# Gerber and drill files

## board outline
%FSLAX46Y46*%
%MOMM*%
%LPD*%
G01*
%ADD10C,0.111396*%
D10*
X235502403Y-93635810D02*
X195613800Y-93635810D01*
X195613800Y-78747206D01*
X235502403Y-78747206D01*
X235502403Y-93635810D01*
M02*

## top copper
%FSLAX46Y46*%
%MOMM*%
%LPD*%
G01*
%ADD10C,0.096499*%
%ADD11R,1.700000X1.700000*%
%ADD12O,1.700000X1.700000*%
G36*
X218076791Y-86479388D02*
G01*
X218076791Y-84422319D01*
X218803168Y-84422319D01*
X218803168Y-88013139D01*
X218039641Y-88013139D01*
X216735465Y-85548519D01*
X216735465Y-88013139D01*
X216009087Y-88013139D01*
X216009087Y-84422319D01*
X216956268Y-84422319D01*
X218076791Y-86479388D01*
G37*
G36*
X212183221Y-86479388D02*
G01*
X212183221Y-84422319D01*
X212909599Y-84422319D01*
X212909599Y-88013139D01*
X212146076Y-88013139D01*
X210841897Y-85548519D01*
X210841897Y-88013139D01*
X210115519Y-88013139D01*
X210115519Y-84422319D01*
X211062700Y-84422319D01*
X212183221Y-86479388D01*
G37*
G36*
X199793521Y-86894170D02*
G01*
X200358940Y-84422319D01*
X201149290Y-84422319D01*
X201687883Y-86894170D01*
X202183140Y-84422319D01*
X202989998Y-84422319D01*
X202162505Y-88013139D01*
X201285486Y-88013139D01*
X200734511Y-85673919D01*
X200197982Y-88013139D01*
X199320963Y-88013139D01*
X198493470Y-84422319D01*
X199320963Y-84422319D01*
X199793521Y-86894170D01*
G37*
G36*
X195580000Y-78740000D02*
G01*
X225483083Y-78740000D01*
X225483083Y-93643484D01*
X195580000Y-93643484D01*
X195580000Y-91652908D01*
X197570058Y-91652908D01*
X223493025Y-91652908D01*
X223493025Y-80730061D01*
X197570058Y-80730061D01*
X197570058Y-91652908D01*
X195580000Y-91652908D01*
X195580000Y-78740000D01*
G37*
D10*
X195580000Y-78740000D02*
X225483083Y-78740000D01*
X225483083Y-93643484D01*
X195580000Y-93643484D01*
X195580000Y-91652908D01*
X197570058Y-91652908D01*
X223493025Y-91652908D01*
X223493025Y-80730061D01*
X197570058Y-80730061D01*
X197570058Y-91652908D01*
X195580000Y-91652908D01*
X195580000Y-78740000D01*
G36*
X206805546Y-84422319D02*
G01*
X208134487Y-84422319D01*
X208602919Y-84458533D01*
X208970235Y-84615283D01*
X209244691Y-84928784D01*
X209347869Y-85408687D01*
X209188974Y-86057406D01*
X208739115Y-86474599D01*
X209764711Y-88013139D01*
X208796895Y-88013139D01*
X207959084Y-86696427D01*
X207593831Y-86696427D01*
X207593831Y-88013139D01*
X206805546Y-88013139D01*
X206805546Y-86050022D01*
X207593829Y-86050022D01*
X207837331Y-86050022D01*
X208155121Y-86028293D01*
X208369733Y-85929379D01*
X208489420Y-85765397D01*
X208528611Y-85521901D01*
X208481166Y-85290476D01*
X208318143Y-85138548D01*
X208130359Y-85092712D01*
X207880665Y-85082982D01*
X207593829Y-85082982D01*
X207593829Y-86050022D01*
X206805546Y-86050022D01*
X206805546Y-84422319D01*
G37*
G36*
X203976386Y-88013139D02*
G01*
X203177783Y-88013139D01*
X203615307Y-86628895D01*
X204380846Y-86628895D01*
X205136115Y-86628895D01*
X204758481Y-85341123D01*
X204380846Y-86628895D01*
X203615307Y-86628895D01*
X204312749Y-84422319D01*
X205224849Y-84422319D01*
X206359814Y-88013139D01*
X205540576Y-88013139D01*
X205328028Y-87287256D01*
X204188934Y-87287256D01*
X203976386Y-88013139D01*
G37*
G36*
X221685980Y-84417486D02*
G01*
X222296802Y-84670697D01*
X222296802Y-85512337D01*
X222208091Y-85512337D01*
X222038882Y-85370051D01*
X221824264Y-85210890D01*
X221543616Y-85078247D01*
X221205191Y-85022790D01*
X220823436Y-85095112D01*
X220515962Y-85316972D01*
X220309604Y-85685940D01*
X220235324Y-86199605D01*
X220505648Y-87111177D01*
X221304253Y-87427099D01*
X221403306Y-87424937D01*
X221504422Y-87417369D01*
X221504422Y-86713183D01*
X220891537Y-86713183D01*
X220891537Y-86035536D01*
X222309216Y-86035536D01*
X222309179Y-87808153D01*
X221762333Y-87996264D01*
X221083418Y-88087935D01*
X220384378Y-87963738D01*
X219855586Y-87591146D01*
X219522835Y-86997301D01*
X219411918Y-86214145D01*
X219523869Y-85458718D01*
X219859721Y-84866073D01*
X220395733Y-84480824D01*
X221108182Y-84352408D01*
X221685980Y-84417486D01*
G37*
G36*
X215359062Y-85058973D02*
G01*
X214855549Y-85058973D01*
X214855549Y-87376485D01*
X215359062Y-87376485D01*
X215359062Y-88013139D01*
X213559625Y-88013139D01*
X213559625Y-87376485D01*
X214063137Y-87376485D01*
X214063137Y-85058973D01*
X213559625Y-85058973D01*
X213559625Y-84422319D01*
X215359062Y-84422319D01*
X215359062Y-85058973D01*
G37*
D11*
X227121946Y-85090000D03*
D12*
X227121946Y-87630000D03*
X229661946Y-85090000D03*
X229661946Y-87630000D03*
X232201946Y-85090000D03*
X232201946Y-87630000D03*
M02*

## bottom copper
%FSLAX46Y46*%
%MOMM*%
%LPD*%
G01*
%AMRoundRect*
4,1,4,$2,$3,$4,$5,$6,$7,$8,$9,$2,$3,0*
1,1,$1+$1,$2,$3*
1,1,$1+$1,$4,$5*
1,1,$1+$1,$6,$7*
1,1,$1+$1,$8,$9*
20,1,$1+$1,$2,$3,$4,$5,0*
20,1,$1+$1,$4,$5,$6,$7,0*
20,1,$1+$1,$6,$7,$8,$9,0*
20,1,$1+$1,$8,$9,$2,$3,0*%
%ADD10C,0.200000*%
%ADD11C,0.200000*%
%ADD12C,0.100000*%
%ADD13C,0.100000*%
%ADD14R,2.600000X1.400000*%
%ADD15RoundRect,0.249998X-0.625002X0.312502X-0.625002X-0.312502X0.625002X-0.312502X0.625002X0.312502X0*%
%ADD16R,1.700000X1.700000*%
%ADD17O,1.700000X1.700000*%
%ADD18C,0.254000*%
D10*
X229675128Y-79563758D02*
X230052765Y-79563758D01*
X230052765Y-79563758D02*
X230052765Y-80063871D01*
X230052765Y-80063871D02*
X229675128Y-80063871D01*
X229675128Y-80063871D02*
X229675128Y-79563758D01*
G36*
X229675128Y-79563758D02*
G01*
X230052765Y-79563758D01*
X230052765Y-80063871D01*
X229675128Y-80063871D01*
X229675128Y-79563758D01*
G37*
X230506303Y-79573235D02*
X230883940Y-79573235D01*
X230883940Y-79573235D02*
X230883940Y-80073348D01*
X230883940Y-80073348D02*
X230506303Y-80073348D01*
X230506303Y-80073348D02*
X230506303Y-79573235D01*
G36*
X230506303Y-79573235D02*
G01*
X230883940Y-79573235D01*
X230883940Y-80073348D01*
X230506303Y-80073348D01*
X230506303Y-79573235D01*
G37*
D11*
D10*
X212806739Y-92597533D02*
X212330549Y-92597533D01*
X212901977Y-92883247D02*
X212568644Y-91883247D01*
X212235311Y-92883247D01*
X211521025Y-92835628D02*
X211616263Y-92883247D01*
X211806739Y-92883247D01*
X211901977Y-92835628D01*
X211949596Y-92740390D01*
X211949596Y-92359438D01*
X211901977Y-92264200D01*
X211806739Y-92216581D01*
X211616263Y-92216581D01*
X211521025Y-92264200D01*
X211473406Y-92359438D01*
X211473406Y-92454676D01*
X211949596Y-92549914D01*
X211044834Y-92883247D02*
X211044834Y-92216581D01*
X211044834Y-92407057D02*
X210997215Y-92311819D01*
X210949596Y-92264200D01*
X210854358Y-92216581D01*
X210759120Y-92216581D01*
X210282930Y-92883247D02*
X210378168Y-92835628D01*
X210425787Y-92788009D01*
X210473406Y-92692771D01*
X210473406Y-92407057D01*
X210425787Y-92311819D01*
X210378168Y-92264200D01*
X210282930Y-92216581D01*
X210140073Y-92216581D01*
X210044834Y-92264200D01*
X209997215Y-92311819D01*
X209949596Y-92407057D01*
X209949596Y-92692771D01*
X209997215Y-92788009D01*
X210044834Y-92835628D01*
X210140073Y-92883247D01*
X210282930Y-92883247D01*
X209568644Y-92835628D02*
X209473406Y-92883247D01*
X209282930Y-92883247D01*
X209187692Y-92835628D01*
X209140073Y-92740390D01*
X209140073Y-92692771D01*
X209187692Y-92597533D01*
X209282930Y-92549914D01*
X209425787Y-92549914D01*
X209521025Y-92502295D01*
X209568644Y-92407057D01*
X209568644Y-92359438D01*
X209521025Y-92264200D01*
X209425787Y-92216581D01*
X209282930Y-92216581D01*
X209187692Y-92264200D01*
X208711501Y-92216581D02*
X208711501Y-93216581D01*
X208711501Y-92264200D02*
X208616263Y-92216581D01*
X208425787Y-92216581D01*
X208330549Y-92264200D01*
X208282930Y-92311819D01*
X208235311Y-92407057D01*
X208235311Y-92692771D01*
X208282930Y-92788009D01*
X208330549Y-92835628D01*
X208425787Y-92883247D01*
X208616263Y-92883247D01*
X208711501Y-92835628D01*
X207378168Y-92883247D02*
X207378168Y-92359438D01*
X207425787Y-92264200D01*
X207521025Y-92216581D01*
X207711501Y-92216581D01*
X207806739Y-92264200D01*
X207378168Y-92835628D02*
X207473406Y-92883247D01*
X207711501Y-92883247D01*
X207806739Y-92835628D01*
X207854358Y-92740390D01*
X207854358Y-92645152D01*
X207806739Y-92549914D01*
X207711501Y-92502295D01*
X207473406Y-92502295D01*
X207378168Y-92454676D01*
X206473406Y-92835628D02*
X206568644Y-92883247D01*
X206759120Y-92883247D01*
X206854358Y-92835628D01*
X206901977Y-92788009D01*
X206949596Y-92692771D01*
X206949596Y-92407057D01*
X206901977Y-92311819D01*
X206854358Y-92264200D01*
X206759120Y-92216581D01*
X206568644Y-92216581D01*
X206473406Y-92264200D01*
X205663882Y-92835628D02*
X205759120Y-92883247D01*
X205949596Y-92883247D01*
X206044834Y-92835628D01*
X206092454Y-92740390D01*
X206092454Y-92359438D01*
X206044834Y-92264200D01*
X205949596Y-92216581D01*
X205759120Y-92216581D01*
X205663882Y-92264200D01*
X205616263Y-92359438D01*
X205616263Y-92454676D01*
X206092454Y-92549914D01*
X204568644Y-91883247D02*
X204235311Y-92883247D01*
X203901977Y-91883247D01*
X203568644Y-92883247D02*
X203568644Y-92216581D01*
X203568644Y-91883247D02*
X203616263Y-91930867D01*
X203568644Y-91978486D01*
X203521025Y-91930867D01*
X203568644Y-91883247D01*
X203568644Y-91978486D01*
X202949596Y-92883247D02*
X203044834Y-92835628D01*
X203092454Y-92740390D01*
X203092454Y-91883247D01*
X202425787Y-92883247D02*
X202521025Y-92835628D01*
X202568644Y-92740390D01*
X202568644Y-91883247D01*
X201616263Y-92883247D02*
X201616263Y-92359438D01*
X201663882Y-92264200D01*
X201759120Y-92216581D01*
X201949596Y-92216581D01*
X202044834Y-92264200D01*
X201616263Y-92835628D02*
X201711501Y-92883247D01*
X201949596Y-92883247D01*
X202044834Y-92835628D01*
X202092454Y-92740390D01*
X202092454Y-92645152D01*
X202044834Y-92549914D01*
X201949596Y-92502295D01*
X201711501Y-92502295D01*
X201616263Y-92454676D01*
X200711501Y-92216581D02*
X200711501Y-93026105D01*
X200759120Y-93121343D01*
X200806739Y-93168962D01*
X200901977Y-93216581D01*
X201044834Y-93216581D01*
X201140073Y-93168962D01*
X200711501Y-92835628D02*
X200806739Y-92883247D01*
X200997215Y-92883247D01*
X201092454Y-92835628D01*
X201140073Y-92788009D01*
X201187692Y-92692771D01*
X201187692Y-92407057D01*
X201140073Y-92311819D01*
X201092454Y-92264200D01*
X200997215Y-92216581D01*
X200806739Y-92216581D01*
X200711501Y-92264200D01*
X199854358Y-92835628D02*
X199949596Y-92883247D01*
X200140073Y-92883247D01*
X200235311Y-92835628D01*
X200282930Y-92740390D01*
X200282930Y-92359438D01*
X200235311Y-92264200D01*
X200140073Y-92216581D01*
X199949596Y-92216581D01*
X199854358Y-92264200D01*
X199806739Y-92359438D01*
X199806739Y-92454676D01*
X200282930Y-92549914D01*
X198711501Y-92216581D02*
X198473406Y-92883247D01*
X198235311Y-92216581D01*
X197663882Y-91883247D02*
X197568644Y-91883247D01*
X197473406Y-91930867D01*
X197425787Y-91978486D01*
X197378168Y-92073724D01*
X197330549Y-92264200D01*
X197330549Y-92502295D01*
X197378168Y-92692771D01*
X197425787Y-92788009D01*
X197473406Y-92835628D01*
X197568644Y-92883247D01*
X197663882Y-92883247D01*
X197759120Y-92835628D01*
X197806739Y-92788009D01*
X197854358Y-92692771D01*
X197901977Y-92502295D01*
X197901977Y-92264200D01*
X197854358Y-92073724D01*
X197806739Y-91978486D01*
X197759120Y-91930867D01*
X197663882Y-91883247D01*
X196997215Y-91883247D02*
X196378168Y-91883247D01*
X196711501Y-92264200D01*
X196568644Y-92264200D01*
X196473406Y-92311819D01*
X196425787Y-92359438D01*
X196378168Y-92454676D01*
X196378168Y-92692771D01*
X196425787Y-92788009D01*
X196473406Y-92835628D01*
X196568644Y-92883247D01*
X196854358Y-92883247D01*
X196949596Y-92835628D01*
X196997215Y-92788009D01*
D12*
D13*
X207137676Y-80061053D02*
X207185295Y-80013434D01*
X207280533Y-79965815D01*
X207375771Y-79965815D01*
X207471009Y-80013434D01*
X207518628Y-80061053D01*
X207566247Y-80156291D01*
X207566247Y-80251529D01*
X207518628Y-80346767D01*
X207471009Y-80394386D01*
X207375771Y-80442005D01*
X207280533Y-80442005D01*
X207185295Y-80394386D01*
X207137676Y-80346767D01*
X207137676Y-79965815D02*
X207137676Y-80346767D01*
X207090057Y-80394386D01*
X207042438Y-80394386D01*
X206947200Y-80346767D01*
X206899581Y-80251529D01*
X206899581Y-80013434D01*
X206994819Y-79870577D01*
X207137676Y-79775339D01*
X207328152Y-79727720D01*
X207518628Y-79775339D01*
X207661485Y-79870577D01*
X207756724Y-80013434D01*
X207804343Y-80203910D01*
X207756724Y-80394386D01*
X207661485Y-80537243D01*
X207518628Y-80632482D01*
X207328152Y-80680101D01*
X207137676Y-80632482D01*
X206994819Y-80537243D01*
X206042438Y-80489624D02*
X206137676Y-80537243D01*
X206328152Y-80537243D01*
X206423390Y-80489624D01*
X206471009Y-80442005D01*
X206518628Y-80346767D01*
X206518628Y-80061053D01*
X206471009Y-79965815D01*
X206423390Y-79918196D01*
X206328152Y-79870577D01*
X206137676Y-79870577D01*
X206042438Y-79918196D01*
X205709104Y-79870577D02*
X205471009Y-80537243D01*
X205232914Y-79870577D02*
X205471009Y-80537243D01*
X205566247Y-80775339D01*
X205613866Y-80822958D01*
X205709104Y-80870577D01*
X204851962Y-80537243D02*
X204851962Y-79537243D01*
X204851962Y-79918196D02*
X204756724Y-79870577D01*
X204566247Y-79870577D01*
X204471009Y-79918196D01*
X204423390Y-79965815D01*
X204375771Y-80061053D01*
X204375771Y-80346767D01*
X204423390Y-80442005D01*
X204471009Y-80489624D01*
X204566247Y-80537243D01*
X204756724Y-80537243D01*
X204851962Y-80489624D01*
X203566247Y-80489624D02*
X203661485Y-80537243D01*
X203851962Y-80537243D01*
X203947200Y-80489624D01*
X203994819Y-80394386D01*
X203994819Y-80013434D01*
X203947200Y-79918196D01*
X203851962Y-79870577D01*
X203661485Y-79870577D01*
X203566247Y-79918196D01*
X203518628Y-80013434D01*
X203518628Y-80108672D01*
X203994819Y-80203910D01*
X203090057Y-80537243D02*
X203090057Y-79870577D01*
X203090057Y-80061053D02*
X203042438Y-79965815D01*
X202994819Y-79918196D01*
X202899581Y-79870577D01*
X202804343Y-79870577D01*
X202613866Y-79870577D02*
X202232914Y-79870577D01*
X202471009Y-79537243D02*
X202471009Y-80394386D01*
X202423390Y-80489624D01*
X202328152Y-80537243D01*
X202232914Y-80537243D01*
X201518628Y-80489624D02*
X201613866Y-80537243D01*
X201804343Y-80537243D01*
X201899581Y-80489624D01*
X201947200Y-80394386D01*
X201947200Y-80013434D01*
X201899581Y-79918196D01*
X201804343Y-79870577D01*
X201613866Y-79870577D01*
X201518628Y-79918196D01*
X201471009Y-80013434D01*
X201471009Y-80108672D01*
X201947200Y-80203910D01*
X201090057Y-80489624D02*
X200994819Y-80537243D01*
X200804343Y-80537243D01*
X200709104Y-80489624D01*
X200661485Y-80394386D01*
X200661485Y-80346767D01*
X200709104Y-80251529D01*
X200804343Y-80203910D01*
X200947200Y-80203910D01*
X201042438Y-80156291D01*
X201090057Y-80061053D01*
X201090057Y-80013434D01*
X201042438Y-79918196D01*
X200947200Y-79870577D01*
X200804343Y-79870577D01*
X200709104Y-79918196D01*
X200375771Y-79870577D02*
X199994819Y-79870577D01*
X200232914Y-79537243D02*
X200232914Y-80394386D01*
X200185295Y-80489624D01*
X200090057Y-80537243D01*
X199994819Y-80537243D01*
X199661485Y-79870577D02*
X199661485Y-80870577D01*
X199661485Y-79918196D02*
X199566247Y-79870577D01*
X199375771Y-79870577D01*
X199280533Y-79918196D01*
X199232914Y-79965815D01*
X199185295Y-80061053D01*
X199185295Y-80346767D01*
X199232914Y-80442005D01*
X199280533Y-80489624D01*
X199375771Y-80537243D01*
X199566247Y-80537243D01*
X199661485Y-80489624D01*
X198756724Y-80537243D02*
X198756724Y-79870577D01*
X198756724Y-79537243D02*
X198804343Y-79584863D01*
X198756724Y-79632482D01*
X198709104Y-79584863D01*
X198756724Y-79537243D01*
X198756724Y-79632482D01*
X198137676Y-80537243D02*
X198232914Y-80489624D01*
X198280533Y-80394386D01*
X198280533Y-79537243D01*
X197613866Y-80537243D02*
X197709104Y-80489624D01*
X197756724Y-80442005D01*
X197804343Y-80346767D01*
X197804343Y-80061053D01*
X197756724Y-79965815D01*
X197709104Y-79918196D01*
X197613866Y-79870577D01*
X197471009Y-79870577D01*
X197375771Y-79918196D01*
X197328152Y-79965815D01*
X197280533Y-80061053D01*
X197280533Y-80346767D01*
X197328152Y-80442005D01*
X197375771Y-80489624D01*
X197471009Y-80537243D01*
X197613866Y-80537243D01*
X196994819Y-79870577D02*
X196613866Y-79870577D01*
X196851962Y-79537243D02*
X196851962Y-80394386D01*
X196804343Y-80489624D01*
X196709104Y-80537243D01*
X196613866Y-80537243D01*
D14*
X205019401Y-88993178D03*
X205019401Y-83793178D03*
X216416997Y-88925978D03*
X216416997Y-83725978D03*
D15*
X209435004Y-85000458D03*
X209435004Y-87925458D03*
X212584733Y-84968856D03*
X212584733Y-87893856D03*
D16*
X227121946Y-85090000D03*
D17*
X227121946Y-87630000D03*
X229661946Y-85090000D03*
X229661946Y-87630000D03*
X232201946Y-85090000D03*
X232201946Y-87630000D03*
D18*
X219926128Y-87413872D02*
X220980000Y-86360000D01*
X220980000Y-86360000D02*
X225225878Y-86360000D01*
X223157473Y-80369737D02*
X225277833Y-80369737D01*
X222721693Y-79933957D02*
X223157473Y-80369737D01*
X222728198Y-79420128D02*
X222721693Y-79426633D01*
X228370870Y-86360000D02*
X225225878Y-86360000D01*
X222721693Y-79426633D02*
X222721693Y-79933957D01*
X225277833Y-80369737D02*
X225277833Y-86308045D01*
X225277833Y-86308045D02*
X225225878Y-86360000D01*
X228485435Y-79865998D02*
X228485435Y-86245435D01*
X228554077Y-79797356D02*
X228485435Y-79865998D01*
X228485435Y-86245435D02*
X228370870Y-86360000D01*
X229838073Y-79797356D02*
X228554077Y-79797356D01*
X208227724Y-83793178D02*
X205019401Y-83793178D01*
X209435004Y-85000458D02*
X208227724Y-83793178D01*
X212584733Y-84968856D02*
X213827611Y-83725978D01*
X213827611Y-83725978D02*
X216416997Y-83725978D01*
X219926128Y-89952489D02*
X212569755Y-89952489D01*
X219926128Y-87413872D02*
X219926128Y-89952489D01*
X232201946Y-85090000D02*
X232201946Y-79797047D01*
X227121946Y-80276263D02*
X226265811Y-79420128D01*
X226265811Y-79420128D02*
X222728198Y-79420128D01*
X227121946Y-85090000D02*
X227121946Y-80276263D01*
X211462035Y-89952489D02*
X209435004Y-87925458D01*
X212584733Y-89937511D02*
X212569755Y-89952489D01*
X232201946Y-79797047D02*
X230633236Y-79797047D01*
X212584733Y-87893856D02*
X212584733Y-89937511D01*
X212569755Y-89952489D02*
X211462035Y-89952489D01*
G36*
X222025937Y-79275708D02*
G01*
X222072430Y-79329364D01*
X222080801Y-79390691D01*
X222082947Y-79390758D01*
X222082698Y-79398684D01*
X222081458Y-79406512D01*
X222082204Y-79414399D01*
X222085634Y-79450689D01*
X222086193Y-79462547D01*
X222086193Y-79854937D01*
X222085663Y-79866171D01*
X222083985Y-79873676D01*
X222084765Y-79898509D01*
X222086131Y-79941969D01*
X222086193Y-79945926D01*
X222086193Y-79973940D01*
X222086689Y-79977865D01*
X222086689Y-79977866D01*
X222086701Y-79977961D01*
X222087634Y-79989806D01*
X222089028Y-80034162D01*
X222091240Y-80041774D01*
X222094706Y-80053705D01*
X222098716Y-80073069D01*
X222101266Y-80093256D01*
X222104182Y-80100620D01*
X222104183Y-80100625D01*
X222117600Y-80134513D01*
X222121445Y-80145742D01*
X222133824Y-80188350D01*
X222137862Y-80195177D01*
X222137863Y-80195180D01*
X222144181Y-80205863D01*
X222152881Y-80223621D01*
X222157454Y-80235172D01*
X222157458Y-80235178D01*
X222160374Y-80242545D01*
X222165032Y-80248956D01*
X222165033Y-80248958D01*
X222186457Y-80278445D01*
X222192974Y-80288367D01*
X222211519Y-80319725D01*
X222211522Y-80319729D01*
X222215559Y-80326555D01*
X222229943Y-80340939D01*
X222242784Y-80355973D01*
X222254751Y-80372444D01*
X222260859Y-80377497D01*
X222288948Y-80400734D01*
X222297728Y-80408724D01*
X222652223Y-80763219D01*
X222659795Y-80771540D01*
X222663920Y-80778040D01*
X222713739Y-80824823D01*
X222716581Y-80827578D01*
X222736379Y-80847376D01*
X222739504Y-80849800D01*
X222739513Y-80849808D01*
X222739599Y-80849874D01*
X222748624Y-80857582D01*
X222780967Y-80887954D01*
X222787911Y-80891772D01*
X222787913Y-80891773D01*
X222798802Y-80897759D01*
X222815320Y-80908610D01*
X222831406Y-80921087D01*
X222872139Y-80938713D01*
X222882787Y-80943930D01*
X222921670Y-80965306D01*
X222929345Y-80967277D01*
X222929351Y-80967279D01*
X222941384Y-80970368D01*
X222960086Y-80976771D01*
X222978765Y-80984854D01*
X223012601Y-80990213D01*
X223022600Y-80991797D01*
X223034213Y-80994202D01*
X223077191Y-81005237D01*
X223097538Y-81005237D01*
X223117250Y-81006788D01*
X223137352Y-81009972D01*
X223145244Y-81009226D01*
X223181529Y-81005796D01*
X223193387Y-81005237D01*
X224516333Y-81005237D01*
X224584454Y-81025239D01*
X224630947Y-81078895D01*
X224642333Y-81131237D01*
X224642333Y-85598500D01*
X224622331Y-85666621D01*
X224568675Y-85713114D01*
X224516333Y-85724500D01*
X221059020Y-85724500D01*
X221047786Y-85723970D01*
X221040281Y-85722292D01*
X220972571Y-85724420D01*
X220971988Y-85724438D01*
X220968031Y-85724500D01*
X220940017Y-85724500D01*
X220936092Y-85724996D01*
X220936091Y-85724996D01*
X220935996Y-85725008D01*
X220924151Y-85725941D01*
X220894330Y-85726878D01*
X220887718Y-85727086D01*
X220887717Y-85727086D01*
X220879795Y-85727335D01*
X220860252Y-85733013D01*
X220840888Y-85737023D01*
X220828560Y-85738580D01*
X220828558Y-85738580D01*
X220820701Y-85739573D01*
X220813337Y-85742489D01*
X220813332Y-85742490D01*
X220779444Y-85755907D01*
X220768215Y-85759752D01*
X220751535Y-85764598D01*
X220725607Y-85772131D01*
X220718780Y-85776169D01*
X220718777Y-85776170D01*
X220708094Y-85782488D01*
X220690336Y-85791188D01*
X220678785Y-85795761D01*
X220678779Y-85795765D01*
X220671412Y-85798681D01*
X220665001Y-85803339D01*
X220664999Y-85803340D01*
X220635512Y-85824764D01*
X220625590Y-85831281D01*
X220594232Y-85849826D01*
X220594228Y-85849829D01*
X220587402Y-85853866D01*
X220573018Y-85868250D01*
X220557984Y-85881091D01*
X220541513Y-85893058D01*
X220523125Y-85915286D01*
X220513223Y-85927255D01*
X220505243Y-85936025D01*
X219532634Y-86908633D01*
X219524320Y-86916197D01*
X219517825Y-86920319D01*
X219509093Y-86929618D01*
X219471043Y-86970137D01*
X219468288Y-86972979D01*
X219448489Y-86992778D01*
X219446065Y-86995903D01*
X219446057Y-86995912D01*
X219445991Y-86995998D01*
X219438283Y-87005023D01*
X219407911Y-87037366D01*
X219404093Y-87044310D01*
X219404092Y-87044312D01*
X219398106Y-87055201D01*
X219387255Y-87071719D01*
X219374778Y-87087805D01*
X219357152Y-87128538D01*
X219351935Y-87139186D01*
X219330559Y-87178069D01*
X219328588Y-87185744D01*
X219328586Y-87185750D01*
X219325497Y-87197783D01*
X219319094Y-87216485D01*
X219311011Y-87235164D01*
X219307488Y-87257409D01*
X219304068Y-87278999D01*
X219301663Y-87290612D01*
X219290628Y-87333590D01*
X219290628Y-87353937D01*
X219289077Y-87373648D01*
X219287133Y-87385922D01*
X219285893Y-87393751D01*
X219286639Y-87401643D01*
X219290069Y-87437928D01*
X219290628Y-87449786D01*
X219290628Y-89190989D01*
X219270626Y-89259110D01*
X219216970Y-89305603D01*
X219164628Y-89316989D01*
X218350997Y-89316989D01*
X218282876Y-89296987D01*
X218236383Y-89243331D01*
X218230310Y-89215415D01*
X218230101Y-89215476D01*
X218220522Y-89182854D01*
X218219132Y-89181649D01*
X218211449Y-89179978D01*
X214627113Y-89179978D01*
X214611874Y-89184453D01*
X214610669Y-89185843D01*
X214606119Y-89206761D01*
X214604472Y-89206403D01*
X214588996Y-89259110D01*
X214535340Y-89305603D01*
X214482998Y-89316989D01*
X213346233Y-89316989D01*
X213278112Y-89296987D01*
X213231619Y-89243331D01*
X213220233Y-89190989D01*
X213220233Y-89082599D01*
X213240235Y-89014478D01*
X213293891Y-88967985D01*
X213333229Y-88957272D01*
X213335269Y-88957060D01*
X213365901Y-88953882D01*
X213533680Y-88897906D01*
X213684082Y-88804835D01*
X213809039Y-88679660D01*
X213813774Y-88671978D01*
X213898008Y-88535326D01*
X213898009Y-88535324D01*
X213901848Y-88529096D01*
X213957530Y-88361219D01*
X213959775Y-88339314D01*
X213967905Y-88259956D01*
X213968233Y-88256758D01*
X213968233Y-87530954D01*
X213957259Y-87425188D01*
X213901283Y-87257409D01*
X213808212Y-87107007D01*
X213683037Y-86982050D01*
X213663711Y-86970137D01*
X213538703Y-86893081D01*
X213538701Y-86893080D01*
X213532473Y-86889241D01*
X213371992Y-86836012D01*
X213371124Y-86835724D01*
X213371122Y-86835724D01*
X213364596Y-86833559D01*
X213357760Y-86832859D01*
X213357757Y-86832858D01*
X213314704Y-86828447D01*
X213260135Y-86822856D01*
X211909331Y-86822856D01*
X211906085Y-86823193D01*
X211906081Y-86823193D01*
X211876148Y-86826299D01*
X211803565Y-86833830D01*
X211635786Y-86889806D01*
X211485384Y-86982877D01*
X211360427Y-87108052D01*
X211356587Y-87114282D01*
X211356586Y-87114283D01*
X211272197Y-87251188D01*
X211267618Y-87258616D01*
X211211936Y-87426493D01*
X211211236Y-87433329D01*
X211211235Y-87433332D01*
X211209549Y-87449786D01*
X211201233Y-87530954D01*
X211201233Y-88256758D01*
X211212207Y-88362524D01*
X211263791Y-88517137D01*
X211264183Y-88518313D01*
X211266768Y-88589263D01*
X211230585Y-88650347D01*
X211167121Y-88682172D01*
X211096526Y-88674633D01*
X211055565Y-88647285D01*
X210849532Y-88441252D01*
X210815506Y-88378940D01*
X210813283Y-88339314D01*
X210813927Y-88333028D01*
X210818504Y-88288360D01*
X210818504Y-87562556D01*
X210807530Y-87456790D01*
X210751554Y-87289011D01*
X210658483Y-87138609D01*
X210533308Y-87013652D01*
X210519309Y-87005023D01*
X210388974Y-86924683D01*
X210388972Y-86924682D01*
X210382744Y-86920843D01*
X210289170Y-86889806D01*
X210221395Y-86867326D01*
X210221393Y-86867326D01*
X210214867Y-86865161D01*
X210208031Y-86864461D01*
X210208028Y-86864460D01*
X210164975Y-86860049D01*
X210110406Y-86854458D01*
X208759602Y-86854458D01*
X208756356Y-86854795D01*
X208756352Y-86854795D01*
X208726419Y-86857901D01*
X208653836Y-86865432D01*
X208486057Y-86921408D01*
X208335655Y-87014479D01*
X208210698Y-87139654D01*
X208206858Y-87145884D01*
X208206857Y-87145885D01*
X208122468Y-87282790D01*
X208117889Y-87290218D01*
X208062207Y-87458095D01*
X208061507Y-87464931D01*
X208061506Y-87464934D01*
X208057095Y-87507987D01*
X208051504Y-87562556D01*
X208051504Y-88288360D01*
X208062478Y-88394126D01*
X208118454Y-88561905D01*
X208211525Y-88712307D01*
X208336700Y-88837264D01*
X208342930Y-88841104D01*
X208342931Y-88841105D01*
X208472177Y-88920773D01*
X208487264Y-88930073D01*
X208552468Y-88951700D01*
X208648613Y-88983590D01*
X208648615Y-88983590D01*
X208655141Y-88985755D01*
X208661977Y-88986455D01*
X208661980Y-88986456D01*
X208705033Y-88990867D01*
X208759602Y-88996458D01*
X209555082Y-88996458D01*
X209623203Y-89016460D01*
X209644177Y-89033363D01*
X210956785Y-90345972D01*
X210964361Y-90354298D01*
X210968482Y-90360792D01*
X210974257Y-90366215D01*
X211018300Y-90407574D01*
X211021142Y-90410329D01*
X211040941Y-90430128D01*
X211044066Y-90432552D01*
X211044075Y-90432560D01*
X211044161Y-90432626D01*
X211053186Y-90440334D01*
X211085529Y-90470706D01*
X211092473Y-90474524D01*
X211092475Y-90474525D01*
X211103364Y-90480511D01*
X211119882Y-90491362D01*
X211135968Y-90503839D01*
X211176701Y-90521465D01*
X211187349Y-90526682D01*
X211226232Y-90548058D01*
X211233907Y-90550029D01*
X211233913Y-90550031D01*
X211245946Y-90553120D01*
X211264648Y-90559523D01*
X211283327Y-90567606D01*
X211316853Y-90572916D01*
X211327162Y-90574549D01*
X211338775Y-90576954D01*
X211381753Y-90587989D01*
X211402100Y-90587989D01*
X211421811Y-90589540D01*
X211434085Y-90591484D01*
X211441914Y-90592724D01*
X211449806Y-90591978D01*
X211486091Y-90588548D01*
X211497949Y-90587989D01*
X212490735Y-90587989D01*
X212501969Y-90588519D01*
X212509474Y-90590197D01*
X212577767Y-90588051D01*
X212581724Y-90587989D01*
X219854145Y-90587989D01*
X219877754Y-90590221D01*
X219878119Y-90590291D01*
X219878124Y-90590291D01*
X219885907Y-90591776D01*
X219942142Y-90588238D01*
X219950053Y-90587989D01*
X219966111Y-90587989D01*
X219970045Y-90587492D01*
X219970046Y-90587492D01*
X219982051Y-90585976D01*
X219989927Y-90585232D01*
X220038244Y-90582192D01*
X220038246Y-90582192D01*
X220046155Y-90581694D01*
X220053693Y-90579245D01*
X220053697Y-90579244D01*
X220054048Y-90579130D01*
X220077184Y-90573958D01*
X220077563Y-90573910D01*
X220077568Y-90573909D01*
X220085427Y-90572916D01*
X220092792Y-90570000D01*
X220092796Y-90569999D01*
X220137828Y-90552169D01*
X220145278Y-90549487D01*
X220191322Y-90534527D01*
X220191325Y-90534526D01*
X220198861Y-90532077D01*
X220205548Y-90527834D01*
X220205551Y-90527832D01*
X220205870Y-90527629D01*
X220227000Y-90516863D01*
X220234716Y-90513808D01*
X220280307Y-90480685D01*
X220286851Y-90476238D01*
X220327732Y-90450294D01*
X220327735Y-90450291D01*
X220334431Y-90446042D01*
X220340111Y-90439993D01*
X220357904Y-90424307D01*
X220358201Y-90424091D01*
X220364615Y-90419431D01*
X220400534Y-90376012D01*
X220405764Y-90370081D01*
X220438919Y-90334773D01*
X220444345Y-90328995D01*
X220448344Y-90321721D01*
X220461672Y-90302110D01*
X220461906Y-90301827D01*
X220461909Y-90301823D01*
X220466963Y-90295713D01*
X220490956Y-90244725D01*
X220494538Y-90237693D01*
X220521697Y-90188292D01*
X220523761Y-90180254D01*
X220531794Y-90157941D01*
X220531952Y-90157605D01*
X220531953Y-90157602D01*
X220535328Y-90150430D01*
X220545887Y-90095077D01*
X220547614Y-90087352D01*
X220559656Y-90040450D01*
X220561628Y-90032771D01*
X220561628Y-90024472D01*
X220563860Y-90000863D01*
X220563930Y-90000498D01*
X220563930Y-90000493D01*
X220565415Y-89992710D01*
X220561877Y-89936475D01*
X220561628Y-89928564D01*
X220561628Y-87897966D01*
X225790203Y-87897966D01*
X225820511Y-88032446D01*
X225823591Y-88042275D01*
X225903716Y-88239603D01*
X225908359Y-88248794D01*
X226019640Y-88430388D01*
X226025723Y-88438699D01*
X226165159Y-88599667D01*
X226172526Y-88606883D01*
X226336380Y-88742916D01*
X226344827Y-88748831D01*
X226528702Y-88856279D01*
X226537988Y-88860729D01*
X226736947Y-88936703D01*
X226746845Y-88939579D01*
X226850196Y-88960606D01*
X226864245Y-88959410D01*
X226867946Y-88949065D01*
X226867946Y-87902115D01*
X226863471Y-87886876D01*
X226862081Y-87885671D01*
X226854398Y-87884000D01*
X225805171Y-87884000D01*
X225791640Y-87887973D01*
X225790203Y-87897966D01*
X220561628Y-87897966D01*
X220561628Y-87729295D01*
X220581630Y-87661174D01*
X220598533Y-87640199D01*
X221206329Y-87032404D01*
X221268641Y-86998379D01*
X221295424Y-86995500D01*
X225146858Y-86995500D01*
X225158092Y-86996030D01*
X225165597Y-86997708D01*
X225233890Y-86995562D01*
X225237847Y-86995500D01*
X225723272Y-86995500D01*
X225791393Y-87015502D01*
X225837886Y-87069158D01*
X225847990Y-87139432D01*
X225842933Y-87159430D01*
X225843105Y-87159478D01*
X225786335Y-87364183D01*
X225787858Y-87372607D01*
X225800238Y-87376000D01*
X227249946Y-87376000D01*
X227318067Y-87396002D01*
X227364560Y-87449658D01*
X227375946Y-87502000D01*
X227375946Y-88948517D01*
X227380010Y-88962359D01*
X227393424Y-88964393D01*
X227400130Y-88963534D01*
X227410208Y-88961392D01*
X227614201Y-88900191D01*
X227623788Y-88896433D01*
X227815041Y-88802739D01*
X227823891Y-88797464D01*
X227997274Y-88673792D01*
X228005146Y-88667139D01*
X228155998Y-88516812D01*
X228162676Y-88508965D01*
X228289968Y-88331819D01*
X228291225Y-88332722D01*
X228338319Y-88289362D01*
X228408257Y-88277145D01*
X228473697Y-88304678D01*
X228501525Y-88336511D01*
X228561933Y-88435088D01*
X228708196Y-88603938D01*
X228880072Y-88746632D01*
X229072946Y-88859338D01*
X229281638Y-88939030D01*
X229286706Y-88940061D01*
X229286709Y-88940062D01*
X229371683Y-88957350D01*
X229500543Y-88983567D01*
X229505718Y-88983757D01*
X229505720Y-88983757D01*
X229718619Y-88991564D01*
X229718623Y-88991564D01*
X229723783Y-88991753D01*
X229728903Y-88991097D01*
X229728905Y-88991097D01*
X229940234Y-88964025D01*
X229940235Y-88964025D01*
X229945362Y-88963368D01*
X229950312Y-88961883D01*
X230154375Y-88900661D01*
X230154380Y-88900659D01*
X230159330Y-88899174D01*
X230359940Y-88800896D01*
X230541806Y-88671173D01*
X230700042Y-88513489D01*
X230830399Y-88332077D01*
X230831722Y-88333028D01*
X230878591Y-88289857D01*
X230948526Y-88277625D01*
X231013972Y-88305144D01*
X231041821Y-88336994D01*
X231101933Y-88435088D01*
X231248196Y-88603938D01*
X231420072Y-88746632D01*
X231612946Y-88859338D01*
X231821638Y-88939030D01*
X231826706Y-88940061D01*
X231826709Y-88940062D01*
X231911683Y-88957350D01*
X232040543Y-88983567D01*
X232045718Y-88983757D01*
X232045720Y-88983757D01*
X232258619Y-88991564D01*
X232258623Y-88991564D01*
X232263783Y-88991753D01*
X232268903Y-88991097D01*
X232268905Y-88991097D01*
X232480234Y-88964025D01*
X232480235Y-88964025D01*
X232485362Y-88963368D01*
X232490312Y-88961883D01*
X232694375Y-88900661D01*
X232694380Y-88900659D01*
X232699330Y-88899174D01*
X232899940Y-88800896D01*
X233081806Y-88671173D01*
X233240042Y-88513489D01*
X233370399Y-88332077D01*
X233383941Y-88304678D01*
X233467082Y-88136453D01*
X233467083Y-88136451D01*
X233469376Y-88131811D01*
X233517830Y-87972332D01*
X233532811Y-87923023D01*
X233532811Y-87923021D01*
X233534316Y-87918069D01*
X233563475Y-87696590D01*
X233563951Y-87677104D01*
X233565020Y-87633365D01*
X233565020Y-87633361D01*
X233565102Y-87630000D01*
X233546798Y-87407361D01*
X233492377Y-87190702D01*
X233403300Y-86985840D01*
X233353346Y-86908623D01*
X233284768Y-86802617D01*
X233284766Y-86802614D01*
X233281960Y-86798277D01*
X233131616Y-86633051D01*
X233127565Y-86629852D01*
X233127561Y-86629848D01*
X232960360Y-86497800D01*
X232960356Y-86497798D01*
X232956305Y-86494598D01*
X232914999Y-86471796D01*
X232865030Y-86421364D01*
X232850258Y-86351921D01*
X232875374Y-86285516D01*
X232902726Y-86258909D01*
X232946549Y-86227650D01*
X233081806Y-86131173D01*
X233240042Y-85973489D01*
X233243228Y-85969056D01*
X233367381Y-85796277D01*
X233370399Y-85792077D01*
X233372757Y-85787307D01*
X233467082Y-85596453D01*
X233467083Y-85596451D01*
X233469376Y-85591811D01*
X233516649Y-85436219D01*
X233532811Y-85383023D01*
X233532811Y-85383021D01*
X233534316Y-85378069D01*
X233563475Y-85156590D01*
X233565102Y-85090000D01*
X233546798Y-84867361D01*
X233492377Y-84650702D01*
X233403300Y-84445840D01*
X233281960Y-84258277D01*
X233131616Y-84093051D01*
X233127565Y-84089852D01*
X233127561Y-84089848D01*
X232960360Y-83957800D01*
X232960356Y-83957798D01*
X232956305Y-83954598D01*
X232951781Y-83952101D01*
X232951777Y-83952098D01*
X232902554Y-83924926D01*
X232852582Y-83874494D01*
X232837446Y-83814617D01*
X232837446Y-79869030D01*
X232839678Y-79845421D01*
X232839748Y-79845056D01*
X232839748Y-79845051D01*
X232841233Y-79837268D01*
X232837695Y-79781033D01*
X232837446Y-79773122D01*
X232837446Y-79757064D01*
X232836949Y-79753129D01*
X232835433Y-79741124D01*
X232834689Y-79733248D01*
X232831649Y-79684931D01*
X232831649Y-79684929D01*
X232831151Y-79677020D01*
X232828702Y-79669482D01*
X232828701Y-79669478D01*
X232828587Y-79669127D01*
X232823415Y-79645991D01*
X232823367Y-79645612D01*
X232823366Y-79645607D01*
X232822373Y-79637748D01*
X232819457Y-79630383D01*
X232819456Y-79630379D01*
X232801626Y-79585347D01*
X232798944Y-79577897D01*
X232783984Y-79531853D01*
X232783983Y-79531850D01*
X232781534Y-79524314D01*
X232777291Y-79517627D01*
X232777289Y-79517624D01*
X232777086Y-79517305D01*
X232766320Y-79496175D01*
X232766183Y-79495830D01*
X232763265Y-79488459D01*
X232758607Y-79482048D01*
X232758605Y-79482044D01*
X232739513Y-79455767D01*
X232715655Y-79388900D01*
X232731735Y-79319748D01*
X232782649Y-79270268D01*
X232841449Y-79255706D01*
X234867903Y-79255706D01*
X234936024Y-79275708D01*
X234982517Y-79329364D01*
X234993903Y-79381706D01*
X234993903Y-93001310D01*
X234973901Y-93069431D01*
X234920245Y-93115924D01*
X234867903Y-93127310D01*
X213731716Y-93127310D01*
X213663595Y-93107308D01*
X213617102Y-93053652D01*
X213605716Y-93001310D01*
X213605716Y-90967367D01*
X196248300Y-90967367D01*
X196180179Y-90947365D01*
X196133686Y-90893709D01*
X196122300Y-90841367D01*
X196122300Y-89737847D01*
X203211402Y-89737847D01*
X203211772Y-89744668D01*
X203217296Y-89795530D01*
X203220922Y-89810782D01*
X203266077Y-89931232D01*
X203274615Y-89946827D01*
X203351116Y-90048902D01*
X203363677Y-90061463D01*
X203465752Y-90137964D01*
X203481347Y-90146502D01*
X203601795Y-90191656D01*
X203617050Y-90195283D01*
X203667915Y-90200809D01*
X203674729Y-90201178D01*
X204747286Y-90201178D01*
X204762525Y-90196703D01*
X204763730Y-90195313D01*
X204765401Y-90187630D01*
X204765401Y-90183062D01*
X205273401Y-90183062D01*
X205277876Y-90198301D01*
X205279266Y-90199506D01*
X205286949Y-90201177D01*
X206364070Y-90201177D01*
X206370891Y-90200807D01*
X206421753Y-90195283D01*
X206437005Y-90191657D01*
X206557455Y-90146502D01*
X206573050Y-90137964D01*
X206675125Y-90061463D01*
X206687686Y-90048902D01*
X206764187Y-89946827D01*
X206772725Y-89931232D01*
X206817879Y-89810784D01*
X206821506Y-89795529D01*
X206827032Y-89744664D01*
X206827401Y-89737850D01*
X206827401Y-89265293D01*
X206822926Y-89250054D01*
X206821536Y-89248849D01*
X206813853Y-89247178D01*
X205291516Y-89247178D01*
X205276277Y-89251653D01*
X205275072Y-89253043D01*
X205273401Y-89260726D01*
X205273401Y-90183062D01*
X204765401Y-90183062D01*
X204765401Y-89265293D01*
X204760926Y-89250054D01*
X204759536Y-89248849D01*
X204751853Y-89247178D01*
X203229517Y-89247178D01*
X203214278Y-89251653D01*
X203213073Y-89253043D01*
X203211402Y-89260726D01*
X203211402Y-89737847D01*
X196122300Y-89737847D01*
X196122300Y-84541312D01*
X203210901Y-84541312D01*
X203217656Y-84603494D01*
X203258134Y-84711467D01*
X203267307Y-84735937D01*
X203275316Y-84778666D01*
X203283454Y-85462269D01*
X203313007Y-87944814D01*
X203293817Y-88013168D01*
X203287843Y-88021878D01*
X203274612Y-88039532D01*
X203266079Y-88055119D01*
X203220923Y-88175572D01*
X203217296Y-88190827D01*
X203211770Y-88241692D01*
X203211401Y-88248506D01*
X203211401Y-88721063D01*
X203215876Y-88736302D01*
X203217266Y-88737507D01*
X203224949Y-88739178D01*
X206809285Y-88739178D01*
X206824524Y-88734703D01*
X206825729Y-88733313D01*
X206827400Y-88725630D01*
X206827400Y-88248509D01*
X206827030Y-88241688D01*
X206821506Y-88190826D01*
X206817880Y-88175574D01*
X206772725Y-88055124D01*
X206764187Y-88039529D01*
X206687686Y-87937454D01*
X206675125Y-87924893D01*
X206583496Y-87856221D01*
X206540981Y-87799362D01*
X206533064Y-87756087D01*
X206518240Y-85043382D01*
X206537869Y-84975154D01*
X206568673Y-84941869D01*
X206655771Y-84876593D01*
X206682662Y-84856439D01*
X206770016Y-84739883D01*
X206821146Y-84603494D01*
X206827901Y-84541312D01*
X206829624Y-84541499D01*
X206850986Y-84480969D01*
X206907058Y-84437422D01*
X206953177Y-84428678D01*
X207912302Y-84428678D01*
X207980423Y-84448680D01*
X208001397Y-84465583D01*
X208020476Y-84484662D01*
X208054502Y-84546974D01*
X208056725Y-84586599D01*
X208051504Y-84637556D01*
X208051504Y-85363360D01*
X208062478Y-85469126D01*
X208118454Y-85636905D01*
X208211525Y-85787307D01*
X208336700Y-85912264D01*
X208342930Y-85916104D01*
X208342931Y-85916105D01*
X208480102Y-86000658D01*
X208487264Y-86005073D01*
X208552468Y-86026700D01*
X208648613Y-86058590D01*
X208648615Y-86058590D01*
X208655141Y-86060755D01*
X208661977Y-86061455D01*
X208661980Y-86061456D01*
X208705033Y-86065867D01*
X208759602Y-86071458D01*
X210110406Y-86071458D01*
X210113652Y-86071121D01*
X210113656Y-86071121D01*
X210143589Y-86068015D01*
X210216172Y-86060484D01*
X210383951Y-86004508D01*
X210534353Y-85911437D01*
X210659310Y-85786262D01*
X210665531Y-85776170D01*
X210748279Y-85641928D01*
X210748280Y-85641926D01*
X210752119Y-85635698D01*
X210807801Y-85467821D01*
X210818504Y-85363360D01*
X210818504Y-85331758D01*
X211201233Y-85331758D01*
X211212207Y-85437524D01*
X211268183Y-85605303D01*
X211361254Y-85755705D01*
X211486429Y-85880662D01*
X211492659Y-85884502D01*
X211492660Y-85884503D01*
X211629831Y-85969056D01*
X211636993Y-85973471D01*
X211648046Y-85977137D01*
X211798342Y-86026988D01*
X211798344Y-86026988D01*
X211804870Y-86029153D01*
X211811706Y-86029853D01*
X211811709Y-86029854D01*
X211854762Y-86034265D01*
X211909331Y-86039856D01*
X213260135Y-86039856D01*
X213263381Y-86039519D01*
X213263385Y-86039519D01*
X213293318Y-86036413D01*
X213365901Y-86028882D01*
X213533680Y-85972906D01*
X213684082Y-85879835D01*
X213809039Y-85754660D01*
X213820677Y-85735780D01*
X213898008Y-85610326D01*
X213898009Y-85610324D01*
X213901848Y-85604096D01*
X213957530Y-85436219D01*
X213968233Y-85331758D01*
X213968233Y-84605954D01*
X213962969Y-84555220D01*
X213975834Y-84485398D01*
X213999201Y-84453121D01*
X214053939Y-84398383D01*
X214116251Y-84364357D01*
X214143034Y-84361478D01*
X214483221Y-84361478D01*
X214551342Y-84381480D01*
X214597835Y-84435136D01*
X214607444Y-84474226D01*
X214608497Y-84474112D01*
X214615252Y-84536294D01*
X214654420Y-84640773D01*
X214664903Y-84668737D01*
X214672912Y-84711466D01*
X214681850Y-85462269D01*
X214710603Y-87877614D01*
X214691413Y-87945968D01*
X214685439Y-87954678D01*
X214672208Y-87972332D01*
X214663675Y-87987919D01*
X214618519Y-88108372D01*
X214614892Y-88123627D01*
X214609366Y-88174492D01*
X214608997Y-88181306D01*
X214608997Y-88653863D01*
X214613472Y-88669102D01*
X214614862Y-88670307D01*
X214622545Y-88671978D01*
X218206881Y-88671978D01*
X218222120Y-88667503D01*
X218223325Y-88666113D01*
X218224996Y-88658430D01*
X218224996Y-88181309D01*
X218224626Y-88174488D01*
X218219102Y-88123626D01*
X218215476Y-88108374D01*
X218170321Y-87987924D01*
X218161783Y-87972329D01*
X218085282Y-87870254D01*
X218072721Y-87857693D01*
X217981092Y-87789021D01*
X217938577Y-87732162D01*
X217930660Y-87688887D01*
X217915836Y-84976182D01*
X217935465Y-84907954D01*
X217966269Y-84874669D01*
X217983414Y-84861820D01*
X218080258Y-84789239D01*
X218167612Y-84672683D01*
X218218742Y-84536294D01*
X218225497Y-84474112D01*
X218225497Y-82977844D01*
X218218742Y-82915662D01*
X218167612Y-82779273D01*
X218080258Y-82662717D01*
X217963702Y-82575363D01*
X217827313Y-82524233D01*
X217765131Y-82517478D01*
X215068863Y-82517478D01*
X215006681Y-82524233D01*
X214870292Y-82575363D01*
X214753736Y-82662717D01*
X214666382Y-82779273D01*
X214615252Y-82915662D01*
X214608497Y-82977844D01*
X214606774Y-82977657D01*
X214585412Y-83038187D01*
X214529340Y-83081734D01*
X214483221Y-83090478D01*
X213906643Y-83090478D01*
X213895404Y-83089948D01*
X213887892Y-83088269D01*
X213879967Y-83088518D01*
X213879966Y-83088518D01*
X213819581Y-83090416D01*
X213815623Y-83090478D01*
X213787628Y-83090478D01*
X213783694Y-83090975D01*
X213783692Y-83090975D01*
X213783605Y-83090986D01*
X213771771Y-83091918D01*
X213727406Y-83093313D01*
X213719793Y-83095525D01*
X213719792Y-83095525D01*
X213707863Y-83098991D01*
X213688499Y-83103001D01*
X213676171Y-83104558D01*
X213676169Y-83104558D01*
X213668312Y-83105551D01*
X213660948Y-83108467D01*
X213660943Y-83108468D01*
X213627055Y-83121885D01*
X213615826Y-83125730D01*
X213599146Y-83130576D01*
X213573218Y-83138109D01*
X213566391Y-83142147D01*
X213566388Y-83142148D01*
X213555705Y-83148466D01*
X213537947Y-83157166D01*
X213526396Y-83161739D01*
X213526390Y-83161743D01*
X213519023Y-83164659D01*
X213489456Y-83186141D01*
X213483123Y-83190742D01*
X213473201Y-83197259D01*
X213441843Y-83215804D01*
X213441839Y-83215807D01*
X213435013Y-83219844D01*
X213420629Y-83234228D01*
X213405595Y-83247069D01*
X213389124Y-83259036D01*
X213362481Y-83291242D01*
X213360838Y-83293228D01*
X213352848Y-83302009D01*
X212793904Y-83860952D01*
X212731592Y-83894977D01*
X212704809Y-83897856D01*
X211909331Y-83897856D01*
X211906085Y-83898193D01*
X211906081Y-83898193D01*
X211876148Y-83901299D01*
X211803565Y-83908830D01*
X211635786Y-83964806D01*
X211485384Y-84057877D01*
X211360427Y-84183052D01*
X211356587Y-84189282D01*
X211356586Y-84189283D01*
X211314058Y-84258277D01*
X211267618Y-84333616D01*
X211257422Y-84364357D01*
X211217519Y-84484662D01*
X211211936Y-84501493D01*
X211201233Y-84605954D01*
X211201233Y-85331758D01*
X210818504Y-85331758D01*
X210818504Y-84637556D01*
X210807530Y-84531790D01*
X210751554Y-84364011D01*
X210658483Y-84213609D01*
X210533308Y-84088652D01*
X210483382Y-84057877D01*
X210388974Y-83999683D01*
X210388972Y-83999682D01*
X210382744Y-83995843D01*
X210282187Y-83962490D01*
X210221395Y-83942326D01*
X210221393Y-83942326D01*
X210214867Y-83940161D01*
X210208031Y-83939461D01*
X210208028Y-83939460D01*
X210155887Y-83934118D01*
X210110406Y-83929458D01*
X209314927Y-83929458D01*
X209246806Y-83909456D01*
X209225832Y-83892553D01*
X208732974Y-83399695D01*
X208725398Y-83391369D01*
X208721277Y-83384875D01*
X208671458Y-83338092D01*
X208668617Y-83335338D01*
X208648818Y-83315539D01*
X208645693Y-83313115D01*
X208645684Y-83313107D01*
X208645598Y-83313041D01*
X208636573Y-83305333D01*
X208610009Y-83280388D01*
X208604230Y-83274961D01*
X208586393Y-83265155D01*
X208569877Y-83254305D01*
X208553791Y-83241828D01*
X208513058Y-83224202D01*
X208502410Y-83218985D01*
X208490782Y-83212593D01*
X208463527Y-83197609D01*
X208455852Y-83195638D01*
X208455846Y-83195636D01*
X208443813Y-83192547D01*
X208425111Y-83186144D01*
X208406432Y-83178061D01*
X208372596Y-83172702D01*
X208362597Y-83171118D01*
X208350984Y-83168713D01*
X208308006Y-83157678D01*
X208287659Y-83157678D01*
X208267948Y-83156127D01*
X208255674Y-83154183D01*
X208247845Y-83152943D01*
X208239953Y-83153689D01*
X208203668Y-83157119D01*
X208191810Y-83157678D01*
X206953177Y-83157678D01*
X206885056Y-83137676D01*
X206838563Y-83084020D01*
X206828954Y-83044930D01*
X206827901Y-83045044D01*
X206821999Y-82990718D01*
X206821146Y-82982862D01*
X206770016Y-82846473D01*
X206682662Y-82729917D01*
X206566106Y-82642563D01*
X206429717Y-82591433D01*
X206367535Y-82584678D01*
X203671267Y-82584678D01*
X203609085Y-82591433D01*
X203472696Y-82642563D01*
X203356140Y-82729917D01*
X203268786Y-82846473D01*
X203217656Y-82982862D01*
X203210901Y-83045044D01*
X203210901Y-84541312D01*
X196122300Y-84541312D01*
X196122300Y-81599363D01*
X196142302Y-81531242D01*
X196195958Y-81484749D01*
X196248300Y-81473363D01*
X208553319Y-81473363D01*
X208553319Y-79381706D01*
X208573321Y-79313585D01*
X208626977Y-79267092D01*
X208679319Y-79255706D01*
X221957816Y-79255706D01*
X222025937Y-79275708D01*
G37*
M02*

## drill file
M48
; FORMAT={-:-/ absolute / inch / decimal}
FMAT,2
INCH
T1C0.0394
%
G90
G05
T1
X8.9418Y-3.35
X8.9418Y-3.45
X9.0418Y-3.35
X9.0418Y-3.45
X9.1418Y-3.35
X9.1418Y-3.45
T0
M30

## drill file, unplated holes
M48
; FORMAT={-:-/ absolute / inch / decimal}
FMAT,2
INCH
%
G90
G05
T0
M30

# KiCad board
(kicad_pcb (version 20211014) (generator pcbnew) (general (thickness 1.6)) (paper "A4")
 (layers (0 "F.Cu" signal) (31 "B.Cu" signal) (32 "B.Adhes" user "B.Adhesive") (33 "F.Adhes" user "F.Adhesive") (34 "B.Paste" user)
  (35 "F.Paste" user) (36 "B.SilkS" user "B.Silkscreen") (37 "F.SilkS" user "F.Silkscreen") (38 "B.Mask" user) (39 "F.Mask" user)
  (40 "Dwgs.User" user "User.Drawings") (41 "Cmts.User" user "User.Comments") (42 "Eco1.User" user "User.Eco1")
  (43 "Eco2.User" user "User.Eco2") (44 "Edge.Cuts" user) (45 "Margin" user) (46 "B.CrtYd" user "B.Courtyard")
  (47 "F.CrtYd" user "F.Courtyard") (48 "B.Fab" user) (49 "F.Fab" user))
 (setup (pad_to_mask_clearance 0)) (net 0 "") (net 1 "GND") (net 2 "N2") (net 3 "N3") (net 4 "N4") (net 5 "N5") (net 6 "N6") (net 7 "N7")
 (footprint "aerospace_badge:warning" (layer "F.Cu") (at 210.82 88.9)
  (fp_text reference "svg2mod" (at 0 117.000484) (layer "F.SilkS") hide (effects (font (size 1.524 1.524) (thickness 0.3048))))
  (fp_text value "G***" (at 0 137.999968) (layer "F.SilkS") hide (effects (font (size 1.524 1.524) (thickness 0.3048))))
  (fp_poly
   (pts (xy 7.983168 -0.886861) (xy 7.219641 -0.886861) (xy 5.915465 -3.351481) (xy 5.915465 -0.886861) (xy 5.189087 -0.886861)
    (xy 5.189087 -4.477681) (xy 6.136268 -4.477681) (xy 7.256791 -2.420612) (xy 7.256791 -4.477681) (xy 7.983168 -4.477681)
    (xy 7.983168 -0.886861))
   (layer "F.Cu") (width 0) (fill solid))
  (fp_poly
   (pts (xy 2.089599 -0.886861) (xy 1.326076 -0.886861) (xy 0.021897 -3.351481) (xy 0.021897 -0.886861) (xy -0.704481 -0.886861)
    (xy -0.704481 -4.477681) (xy 0.2427 -4.477681) (xy 1.363221 -2.420612) (xy 1.363221 -4.477681) (xy 2.089599 -4.477681)
    (xy 2.089599 -0.886861))
   (layer "F.Cu") (width 0) (fill solid))
  (fp_poly
   (pts (xy -7.830002 -4.477681) (xy -8.657495 -0.886861) (xy -9.534514 -0.886861) (xy -10.085489 -3.226081) (xy -10.622018 -0.886861)
    (xy -11.499037 -0.886861) (xy -12.32653 -4.477681) (xy -11.499037 -4.477681) (xy -11.026479 -2.00583) (xy -10.46106 -4.477681)
    (xy -9.67071 -4.477681) (xy -9.132117 -2.00583) (xy -8.63686 -4.477681) (xy -7.830002 -4.477681))
   (layer "F.Cu") (width 0) (fill solid))
  (fp_poly
   (pts (xy -15.24 -10.16) (xy -15.24 4.743484) (xy 12.673025 4.743484) (xy 12.673025 2.752908) (xy -13.249942 2.752908)
    (xy -13.249942 -8.169939) (xy 12.673025 -8.169939) (xy 12.673025 2.752908) (xy 12.673025 4.743484) (xy 14.663083 4.743484)
    (xy 14.663083 -10.16) (xy -15.24 -10.16))
   (layer "F.Cu") (width 0.096499) (fill solid))
  (fp_poly
   (pts (xy -1.055289 -0.886861) (xy -2.023105 -0.886861) (xy -2.860916 -2.203573) (xy -3.226169 -2.203573) (xy -3.226169 -0.886861)
    (xy -3.226171 -0.886861) (xy -3.226171 -2.849978) (xy -2.982669 -2.849978) (xy -2.664879 -2.871707) (xy -2.450267 -2.970621)
    (xy -2.33058 -3.134603) (xy -2.291377 -3.378171) (xy -2.29137 -3.378009) (xy -2.338834 -3.609524) (xy -2.501857 -3.761452)
    (xy -2.689641 -3.807288) (xy -2.939335 -3.817018) (xy -3.226171 -3.817018) (xy -3.226171 -2.849978) (xy -3.226171 -0.886861)
    (xy -4.014454 -0.886861) (xy -4.014454 -4.477681) (xy -2.685513 -4.477681) (xy -2.217081 -4.441467) (xy -1.849765 -4.284717)
    (xy -1.575309 -3.971216) (xy -1.472131 -3.491313) (xy -1.631026 -2.842594) (xy -2.080885 -2.425401) (xy -1.055289 -0.886861))
   (layer "F.Cu") (width 0) (fill solid))
  (fp_poly
   (pts (xy -4.460186 -0.886861) (xy -5.279424 -0.886861) (xy -5.491972 -1.612744) (xy -5.683885 -1.612744) (xy -5.683885 -2.271105)
    (xy -6.061519 -3.558877) (xy -6.439154 -2.271105) (xy -5.683885 -2.271105) (xy -5.683885 -1.612744) (xy -6.631066 -1.612744)
    (xy -6.843614 -0.886861) (xy -7.642217 -0.886861) (xy -6.507251 -4.477681) (xy -5.595151 -4.477681) (xy -4.460186 -0.886861))
   (layer "F.Cu") (width 0) (fill solid))
  (fp_poly
   (pts (xy 11.489179 -1.091847) (xy 10.942333 -0.903736) (xy 10.263418 -0.812065) (xy 9.564378 -0.936262) (xy 9.035586 -1.308854)
    (xy 8.702835 -1.902699) (xy 8.591918 -2.685855) (xy 8.703869 -3.441282) (xy 9.039721 -4.033927) (xy 9.575733 -4.419176)
    (xy 10.288182 -4.547592) (xy 10.86598 -4.482514) (xy 11.476802 -4.229303) (xy 11.476802 -3.387663) (xy 11.388091 -3.387663)
    (xy 11.218882 -3.529949) (xy 11.004264 -3.68911) (xy 10.723616 -3.821753) (xy 10.385191 -3.87721) (xy 10.003436 -3.804888)
    (xy 9.695962 -3.583028) (xy 9.489604 -3.21406) (xy 9.415324 -2.700395) (xy 9.685648 -1.788823) (xy 10.484253 -1.472901)
    (xy 10.583306 -1.475063) (xy 10.684422 -1.482631) (xy 10.684422 -2.186817) (xy 10.071537 -2.186817) (xy 10.071537 -2.864464)
    (xy 11.489216 -2.864464) (xy 11.489179 -1.091847))
   (layer "F.Cu") (width 0) (fill solid))
  (fp_poly
   (pts (xy 4.539062 -0.886861) (xy 2.739625 -0.886861) (xy 2.739625 -1.523515) (xy 3.243137 -1.523515) (xy 3.243137 -3.841027)
    (xy 2.739625 -3.841027) (xy 2.739625 -4.477681) (xy 4.539062 -4.477681) (xy 4.539062 -3.841027) (xy 4.035549 -3.841027)
    (xy 4.035549 -1.523515) (xy 4.539062 -1.523515) (xy 4.539062 -0.886861))
   (layer "F.Cu") (width 0) (fill solid))
  (fp_poly
   (pts (xy -15.2062 -10.152794) (xy -15.2062 4.73581) (xy 24.682403 4.73581) (xy 24.682403 -10.152794) (xy -15.2062 -10.152794))
   (layer "Edge.Cuts") (width 0.111396) (fill none)))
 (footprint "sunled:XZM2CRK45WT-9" (layer "B.Cu") (at 205.019401 86.393178 90)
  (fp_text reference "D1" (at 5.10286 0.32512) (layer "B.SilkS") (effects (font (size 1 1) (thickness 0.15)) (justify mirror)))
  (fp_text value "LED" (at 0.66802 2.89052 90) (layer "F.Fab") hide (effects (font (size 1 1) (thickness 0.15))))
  (pad "1" smd rect (at -2.6 0 90) (size 1.4 2.6) (layers "B.Cu" "B.Paste" "B.Mask") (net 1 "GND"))
  (pad "2" smd rect (at 2.6 0 90) (size 1.4 2.6) (layers "B.Cu" "B.Paste" "B.Mask") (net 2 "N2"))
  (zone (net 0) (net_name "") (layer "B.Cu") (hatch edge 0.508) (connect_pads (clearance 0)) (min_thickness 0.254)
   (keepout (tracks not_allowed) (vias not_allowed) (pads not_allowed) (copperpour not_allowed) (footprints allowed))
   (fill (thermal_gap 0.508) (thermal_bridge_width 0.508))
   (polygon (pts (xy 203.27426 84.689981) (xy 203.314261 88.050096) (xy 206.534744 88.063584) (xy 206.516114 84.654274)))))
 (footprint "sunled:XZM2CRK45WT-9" (layer "B.Cu") (at 216.416997 86.325978 90)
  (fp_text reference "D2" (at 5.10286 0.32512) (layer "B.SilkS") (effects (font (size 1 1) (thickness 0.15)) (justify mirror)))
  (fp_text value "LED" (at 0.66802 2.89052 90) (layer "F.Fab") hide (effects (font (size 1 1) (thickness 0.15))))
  (pad "1" smd rect (at -2.6 0 90) (size 1.4 2.6) (layers "B.Cu" "B.Paste" "B.Mask") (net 1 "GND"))
  (pad "2" smd rect (at 2.6 0 90) (size 1.4 2.6) (layers "B.Cu" "B.Paste" "B.Mask") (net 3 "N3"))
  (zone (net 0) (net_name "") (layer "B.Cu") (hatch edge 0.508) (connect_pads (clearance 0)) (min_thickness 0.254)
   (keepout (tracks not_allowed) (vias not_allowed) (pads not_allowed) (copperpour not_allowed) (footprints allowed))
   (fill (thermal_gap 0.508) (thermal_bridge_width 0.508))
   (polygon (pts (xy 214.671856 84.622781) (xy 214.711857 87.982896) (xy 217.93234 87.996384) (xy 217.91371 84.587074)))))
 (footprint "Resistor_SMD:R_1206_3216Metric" (layer "B.Cu") (at 209.435004 86.462958 -90)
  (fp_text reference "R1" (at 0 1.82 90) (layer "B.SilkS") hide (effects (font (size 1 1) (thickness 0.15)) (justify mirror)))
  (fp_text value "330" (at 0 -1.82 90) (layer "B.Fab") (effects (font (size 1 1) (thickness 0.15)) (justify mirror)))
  (pad "1" smd roundrect locked (at -1.4625 0 270) (size 1.125 1.75) (layers "B.Cu" "B.Paste" "B.Mask") (roundrect_rratio 0.2222204444)
   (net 2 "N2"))
  (pad "2" smd roundrect locked (at 1.4625 0 270) (size 1.125 1.75) (layers "B.Cu" "B.Paste" "B.Mask") (roundrect_rratio 0.2222204444)
   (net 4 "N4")))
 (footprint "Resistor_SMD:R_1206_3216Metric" (layer "B.Cu") (at 212.584733 86.431356 -90)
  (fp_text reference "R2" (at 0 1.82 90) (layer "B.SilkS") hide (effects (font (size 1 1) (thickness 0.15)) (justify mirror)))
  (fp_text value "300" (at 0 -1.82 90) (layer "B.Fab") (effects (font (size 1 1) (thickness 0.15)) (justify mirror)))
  (pad "1" smd roundrect locked (at -1.4625 0 270) (size 1.125 1.75) (layers "B.Cu" "B.Paste" "B.Mask") (roundrect_rratio 0.2222204444)
   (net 3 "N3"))
  (pad "2" smd roundrect locked (at 1.4625 0 270) (size 1.125 1.75) (layers "B.Cu" "B.Paste" "B.Mask") (roundrect_rratio 0.2222204444)
   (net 4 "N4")))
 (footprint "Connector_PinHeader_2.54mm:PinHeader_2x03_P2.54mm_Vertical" (layer "B.Cu") (at 227.121946 85.09 -90)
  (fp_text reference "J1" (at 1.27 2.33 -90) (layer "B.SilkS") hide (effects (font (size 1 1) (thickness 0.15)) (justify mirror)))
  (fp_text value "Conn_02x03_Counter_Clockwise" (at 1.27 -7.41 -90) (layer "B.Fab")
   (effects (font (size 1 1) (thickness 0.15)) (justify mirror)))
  (pad "1" thru_hole rect locked (at 0 0 270) (size 1.7 1.7) (drill 1) (layers *.Cu *.Mask) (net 4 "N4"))
  (pad "2" thru_hole oval locked (at 2.54 0 270) (size 1.7 1.7) (drill 1) (layers *.Cu *.Mask) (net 1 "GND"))
  (pad "3" thru_hole oval locked (at 0 -2.54 270) (size 1.7 1.7) (drill 1) (layers *.Cu *.Mask) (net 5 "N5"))
  (pad "4" thru_hole oval locked (at 2.54 -2.54 270) (size 1.7 1.7) (drill 1) (layers *.Cu *.Mask) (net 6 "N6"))
  (pad "5" thru_hole oval locked (at 0 -5.08 270) (size 1.7 1.7) (drill 1) (layers *.Cu *.Mask) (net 4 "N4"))
  (pad "6" thru_hole oval locked (at 2.54 -5.08 270) (size 1.7 1.7) (drill 1) (layers *.Cu *.Mask) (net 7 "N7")))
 (gr_rect (start 229.675128 79.563758) (end 230.052765 80.063871) (layer "B.Cu") (width 0.2) (fill solid))
 (gr_rect (start 230.506303 79.573235) (end 230.88394 80.073348) (layer "B.Cu") (width 0.2) (fill solid))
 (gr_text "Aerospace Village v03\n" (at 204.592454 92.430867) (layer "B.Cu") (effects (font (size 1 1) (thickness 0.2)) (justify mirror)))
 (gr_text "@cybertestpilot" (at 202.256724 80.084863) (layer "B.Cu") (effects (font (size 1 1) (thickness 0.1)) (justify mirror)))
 (segment (start 208.227724 83.793178) (end 205.019401 83.793178) (width 0.254) (layer "B.Cu") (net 2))
 (segment (start 209.435004 85.000458) (end 208.227724 83.793178) (width 0.254) (layer "B.Cu") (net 2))
 (segment (start 212.584733 84.968856) (end 213.827611 83.725978) (width 0.254) (layer "B.Cu") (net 3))
 (segment (start 213.827611 83.725978) (end 216.416997 83.725978) (width 0.254) (layer "B.Cu") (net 3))
 (segment (start 219.926128 89.952489) (end 212.569755 89.952489) (width 0.254) (layer "B.Cu") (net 4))
 (segment (start 228.485435 79.865998) (end 228.485435 86.245435) (width 0.254) (layer "B.Cu") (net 4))
 (segment (start 219.926128 87.413872) (end 219.926128 89.952489) (width 0.254) (layer "B.Cu") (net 4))
 (segment (start 220.98 86.36) (end 225.225878 86.36) (width 0.254) (layer "B.Cu") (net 4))
 (segment (start 232.201946 85.09) (end 232.201946 79.797047) (width 0.254) (layer "B.Cu") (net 4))
 (segment (start 228.485435 86.245435) (end 228.37087 86.36) (width 0.254) (layer "B.Cu") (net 4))
 (segment (start 227.121946 80.276263) (end 226.265811 79.420128) (width 0.254) (layer "B.Cu") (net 4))
 (segment (start 228.37087 86.36) (end 225.225878 86.36) (width 0.254) (layer "B.Cu") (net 4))
 (segment (start 222.721693 79.933957) (end 223.157473 80.369737) (width 0.254) (layer "B.Cu") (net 4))
 (segment (start 225.277833 86.308045) (end 225.225878 86.36) (width 0.254) (layer "B.Cu") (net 4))
 (segment (start 222.728198 79.420128) (end 222.721693 79.426633) (width 0.254) (layer "B.Cu") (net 4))
 (segment (start 226.265811 79.420128) (end 222.728198 79.420128) (width 0.254) (layer "B.Cu") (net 4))
 (segment (start 227.121946 85.09) (end 227.121946 80.276263) (width 0.254) (layer "B.Cu") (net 4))
 (segment (start 225.277833 80.369737) (end 225.277833 86.308045) (width 0.254) (layer "B.Cu") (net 4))
 (segment (start 219.926128 87.413872) (end 220.98 86.36) (width 0.254) (layer "B.Cu") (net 4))
 (segment (start 228.554077 79.797356) (end 228.485435 79.865998) (width 0.254) (layer "B.Cu") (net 4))
 (segment (start 211.462035 89.952489) (end 209.435004 87.925458) (width 0.254) (layer "B.Cu") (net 4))
 (segment (start 212.584733 89.937511) (end 212.569755 89.952489) (width 0.254) (layer "B.Cu") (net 4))
 (segment (start 229.838073 79.797356) (end 228.554077 79.797356) (width 0.254) (layer "B.Cu") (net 4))
 (segment (start 222.721693 79.426633) (end 222.721693 79.933957) (width 0.254) (layer "B.Cu") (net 4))
 (segment (start 232.201946 79.797047) (end 230.633236 79.797047) (width 0.254) (layer "B.Cu") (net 4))
 (segment (start 212.584733 87.893856) (end 212.584733 89.937511) (width 0.254) (layer "B.Cu") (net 4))
 (segment (start 212.569755 89.952489) (end 211.462035 89.952489) (width 0.254) (layer "B.Cu") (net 4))
 (segment (start 223.157473 80.369737) (end 225.277833 80.369737) (width 0.254) (layer "B.Cu") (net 4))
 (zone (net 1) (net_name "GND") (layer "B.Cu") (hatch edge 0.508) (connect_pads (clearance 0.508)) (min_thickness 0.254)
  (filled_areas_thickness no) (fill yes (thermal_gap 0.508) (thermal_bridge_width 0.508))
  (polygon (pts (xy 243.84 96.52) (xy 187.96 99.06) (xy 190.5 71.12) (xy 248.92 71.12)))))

